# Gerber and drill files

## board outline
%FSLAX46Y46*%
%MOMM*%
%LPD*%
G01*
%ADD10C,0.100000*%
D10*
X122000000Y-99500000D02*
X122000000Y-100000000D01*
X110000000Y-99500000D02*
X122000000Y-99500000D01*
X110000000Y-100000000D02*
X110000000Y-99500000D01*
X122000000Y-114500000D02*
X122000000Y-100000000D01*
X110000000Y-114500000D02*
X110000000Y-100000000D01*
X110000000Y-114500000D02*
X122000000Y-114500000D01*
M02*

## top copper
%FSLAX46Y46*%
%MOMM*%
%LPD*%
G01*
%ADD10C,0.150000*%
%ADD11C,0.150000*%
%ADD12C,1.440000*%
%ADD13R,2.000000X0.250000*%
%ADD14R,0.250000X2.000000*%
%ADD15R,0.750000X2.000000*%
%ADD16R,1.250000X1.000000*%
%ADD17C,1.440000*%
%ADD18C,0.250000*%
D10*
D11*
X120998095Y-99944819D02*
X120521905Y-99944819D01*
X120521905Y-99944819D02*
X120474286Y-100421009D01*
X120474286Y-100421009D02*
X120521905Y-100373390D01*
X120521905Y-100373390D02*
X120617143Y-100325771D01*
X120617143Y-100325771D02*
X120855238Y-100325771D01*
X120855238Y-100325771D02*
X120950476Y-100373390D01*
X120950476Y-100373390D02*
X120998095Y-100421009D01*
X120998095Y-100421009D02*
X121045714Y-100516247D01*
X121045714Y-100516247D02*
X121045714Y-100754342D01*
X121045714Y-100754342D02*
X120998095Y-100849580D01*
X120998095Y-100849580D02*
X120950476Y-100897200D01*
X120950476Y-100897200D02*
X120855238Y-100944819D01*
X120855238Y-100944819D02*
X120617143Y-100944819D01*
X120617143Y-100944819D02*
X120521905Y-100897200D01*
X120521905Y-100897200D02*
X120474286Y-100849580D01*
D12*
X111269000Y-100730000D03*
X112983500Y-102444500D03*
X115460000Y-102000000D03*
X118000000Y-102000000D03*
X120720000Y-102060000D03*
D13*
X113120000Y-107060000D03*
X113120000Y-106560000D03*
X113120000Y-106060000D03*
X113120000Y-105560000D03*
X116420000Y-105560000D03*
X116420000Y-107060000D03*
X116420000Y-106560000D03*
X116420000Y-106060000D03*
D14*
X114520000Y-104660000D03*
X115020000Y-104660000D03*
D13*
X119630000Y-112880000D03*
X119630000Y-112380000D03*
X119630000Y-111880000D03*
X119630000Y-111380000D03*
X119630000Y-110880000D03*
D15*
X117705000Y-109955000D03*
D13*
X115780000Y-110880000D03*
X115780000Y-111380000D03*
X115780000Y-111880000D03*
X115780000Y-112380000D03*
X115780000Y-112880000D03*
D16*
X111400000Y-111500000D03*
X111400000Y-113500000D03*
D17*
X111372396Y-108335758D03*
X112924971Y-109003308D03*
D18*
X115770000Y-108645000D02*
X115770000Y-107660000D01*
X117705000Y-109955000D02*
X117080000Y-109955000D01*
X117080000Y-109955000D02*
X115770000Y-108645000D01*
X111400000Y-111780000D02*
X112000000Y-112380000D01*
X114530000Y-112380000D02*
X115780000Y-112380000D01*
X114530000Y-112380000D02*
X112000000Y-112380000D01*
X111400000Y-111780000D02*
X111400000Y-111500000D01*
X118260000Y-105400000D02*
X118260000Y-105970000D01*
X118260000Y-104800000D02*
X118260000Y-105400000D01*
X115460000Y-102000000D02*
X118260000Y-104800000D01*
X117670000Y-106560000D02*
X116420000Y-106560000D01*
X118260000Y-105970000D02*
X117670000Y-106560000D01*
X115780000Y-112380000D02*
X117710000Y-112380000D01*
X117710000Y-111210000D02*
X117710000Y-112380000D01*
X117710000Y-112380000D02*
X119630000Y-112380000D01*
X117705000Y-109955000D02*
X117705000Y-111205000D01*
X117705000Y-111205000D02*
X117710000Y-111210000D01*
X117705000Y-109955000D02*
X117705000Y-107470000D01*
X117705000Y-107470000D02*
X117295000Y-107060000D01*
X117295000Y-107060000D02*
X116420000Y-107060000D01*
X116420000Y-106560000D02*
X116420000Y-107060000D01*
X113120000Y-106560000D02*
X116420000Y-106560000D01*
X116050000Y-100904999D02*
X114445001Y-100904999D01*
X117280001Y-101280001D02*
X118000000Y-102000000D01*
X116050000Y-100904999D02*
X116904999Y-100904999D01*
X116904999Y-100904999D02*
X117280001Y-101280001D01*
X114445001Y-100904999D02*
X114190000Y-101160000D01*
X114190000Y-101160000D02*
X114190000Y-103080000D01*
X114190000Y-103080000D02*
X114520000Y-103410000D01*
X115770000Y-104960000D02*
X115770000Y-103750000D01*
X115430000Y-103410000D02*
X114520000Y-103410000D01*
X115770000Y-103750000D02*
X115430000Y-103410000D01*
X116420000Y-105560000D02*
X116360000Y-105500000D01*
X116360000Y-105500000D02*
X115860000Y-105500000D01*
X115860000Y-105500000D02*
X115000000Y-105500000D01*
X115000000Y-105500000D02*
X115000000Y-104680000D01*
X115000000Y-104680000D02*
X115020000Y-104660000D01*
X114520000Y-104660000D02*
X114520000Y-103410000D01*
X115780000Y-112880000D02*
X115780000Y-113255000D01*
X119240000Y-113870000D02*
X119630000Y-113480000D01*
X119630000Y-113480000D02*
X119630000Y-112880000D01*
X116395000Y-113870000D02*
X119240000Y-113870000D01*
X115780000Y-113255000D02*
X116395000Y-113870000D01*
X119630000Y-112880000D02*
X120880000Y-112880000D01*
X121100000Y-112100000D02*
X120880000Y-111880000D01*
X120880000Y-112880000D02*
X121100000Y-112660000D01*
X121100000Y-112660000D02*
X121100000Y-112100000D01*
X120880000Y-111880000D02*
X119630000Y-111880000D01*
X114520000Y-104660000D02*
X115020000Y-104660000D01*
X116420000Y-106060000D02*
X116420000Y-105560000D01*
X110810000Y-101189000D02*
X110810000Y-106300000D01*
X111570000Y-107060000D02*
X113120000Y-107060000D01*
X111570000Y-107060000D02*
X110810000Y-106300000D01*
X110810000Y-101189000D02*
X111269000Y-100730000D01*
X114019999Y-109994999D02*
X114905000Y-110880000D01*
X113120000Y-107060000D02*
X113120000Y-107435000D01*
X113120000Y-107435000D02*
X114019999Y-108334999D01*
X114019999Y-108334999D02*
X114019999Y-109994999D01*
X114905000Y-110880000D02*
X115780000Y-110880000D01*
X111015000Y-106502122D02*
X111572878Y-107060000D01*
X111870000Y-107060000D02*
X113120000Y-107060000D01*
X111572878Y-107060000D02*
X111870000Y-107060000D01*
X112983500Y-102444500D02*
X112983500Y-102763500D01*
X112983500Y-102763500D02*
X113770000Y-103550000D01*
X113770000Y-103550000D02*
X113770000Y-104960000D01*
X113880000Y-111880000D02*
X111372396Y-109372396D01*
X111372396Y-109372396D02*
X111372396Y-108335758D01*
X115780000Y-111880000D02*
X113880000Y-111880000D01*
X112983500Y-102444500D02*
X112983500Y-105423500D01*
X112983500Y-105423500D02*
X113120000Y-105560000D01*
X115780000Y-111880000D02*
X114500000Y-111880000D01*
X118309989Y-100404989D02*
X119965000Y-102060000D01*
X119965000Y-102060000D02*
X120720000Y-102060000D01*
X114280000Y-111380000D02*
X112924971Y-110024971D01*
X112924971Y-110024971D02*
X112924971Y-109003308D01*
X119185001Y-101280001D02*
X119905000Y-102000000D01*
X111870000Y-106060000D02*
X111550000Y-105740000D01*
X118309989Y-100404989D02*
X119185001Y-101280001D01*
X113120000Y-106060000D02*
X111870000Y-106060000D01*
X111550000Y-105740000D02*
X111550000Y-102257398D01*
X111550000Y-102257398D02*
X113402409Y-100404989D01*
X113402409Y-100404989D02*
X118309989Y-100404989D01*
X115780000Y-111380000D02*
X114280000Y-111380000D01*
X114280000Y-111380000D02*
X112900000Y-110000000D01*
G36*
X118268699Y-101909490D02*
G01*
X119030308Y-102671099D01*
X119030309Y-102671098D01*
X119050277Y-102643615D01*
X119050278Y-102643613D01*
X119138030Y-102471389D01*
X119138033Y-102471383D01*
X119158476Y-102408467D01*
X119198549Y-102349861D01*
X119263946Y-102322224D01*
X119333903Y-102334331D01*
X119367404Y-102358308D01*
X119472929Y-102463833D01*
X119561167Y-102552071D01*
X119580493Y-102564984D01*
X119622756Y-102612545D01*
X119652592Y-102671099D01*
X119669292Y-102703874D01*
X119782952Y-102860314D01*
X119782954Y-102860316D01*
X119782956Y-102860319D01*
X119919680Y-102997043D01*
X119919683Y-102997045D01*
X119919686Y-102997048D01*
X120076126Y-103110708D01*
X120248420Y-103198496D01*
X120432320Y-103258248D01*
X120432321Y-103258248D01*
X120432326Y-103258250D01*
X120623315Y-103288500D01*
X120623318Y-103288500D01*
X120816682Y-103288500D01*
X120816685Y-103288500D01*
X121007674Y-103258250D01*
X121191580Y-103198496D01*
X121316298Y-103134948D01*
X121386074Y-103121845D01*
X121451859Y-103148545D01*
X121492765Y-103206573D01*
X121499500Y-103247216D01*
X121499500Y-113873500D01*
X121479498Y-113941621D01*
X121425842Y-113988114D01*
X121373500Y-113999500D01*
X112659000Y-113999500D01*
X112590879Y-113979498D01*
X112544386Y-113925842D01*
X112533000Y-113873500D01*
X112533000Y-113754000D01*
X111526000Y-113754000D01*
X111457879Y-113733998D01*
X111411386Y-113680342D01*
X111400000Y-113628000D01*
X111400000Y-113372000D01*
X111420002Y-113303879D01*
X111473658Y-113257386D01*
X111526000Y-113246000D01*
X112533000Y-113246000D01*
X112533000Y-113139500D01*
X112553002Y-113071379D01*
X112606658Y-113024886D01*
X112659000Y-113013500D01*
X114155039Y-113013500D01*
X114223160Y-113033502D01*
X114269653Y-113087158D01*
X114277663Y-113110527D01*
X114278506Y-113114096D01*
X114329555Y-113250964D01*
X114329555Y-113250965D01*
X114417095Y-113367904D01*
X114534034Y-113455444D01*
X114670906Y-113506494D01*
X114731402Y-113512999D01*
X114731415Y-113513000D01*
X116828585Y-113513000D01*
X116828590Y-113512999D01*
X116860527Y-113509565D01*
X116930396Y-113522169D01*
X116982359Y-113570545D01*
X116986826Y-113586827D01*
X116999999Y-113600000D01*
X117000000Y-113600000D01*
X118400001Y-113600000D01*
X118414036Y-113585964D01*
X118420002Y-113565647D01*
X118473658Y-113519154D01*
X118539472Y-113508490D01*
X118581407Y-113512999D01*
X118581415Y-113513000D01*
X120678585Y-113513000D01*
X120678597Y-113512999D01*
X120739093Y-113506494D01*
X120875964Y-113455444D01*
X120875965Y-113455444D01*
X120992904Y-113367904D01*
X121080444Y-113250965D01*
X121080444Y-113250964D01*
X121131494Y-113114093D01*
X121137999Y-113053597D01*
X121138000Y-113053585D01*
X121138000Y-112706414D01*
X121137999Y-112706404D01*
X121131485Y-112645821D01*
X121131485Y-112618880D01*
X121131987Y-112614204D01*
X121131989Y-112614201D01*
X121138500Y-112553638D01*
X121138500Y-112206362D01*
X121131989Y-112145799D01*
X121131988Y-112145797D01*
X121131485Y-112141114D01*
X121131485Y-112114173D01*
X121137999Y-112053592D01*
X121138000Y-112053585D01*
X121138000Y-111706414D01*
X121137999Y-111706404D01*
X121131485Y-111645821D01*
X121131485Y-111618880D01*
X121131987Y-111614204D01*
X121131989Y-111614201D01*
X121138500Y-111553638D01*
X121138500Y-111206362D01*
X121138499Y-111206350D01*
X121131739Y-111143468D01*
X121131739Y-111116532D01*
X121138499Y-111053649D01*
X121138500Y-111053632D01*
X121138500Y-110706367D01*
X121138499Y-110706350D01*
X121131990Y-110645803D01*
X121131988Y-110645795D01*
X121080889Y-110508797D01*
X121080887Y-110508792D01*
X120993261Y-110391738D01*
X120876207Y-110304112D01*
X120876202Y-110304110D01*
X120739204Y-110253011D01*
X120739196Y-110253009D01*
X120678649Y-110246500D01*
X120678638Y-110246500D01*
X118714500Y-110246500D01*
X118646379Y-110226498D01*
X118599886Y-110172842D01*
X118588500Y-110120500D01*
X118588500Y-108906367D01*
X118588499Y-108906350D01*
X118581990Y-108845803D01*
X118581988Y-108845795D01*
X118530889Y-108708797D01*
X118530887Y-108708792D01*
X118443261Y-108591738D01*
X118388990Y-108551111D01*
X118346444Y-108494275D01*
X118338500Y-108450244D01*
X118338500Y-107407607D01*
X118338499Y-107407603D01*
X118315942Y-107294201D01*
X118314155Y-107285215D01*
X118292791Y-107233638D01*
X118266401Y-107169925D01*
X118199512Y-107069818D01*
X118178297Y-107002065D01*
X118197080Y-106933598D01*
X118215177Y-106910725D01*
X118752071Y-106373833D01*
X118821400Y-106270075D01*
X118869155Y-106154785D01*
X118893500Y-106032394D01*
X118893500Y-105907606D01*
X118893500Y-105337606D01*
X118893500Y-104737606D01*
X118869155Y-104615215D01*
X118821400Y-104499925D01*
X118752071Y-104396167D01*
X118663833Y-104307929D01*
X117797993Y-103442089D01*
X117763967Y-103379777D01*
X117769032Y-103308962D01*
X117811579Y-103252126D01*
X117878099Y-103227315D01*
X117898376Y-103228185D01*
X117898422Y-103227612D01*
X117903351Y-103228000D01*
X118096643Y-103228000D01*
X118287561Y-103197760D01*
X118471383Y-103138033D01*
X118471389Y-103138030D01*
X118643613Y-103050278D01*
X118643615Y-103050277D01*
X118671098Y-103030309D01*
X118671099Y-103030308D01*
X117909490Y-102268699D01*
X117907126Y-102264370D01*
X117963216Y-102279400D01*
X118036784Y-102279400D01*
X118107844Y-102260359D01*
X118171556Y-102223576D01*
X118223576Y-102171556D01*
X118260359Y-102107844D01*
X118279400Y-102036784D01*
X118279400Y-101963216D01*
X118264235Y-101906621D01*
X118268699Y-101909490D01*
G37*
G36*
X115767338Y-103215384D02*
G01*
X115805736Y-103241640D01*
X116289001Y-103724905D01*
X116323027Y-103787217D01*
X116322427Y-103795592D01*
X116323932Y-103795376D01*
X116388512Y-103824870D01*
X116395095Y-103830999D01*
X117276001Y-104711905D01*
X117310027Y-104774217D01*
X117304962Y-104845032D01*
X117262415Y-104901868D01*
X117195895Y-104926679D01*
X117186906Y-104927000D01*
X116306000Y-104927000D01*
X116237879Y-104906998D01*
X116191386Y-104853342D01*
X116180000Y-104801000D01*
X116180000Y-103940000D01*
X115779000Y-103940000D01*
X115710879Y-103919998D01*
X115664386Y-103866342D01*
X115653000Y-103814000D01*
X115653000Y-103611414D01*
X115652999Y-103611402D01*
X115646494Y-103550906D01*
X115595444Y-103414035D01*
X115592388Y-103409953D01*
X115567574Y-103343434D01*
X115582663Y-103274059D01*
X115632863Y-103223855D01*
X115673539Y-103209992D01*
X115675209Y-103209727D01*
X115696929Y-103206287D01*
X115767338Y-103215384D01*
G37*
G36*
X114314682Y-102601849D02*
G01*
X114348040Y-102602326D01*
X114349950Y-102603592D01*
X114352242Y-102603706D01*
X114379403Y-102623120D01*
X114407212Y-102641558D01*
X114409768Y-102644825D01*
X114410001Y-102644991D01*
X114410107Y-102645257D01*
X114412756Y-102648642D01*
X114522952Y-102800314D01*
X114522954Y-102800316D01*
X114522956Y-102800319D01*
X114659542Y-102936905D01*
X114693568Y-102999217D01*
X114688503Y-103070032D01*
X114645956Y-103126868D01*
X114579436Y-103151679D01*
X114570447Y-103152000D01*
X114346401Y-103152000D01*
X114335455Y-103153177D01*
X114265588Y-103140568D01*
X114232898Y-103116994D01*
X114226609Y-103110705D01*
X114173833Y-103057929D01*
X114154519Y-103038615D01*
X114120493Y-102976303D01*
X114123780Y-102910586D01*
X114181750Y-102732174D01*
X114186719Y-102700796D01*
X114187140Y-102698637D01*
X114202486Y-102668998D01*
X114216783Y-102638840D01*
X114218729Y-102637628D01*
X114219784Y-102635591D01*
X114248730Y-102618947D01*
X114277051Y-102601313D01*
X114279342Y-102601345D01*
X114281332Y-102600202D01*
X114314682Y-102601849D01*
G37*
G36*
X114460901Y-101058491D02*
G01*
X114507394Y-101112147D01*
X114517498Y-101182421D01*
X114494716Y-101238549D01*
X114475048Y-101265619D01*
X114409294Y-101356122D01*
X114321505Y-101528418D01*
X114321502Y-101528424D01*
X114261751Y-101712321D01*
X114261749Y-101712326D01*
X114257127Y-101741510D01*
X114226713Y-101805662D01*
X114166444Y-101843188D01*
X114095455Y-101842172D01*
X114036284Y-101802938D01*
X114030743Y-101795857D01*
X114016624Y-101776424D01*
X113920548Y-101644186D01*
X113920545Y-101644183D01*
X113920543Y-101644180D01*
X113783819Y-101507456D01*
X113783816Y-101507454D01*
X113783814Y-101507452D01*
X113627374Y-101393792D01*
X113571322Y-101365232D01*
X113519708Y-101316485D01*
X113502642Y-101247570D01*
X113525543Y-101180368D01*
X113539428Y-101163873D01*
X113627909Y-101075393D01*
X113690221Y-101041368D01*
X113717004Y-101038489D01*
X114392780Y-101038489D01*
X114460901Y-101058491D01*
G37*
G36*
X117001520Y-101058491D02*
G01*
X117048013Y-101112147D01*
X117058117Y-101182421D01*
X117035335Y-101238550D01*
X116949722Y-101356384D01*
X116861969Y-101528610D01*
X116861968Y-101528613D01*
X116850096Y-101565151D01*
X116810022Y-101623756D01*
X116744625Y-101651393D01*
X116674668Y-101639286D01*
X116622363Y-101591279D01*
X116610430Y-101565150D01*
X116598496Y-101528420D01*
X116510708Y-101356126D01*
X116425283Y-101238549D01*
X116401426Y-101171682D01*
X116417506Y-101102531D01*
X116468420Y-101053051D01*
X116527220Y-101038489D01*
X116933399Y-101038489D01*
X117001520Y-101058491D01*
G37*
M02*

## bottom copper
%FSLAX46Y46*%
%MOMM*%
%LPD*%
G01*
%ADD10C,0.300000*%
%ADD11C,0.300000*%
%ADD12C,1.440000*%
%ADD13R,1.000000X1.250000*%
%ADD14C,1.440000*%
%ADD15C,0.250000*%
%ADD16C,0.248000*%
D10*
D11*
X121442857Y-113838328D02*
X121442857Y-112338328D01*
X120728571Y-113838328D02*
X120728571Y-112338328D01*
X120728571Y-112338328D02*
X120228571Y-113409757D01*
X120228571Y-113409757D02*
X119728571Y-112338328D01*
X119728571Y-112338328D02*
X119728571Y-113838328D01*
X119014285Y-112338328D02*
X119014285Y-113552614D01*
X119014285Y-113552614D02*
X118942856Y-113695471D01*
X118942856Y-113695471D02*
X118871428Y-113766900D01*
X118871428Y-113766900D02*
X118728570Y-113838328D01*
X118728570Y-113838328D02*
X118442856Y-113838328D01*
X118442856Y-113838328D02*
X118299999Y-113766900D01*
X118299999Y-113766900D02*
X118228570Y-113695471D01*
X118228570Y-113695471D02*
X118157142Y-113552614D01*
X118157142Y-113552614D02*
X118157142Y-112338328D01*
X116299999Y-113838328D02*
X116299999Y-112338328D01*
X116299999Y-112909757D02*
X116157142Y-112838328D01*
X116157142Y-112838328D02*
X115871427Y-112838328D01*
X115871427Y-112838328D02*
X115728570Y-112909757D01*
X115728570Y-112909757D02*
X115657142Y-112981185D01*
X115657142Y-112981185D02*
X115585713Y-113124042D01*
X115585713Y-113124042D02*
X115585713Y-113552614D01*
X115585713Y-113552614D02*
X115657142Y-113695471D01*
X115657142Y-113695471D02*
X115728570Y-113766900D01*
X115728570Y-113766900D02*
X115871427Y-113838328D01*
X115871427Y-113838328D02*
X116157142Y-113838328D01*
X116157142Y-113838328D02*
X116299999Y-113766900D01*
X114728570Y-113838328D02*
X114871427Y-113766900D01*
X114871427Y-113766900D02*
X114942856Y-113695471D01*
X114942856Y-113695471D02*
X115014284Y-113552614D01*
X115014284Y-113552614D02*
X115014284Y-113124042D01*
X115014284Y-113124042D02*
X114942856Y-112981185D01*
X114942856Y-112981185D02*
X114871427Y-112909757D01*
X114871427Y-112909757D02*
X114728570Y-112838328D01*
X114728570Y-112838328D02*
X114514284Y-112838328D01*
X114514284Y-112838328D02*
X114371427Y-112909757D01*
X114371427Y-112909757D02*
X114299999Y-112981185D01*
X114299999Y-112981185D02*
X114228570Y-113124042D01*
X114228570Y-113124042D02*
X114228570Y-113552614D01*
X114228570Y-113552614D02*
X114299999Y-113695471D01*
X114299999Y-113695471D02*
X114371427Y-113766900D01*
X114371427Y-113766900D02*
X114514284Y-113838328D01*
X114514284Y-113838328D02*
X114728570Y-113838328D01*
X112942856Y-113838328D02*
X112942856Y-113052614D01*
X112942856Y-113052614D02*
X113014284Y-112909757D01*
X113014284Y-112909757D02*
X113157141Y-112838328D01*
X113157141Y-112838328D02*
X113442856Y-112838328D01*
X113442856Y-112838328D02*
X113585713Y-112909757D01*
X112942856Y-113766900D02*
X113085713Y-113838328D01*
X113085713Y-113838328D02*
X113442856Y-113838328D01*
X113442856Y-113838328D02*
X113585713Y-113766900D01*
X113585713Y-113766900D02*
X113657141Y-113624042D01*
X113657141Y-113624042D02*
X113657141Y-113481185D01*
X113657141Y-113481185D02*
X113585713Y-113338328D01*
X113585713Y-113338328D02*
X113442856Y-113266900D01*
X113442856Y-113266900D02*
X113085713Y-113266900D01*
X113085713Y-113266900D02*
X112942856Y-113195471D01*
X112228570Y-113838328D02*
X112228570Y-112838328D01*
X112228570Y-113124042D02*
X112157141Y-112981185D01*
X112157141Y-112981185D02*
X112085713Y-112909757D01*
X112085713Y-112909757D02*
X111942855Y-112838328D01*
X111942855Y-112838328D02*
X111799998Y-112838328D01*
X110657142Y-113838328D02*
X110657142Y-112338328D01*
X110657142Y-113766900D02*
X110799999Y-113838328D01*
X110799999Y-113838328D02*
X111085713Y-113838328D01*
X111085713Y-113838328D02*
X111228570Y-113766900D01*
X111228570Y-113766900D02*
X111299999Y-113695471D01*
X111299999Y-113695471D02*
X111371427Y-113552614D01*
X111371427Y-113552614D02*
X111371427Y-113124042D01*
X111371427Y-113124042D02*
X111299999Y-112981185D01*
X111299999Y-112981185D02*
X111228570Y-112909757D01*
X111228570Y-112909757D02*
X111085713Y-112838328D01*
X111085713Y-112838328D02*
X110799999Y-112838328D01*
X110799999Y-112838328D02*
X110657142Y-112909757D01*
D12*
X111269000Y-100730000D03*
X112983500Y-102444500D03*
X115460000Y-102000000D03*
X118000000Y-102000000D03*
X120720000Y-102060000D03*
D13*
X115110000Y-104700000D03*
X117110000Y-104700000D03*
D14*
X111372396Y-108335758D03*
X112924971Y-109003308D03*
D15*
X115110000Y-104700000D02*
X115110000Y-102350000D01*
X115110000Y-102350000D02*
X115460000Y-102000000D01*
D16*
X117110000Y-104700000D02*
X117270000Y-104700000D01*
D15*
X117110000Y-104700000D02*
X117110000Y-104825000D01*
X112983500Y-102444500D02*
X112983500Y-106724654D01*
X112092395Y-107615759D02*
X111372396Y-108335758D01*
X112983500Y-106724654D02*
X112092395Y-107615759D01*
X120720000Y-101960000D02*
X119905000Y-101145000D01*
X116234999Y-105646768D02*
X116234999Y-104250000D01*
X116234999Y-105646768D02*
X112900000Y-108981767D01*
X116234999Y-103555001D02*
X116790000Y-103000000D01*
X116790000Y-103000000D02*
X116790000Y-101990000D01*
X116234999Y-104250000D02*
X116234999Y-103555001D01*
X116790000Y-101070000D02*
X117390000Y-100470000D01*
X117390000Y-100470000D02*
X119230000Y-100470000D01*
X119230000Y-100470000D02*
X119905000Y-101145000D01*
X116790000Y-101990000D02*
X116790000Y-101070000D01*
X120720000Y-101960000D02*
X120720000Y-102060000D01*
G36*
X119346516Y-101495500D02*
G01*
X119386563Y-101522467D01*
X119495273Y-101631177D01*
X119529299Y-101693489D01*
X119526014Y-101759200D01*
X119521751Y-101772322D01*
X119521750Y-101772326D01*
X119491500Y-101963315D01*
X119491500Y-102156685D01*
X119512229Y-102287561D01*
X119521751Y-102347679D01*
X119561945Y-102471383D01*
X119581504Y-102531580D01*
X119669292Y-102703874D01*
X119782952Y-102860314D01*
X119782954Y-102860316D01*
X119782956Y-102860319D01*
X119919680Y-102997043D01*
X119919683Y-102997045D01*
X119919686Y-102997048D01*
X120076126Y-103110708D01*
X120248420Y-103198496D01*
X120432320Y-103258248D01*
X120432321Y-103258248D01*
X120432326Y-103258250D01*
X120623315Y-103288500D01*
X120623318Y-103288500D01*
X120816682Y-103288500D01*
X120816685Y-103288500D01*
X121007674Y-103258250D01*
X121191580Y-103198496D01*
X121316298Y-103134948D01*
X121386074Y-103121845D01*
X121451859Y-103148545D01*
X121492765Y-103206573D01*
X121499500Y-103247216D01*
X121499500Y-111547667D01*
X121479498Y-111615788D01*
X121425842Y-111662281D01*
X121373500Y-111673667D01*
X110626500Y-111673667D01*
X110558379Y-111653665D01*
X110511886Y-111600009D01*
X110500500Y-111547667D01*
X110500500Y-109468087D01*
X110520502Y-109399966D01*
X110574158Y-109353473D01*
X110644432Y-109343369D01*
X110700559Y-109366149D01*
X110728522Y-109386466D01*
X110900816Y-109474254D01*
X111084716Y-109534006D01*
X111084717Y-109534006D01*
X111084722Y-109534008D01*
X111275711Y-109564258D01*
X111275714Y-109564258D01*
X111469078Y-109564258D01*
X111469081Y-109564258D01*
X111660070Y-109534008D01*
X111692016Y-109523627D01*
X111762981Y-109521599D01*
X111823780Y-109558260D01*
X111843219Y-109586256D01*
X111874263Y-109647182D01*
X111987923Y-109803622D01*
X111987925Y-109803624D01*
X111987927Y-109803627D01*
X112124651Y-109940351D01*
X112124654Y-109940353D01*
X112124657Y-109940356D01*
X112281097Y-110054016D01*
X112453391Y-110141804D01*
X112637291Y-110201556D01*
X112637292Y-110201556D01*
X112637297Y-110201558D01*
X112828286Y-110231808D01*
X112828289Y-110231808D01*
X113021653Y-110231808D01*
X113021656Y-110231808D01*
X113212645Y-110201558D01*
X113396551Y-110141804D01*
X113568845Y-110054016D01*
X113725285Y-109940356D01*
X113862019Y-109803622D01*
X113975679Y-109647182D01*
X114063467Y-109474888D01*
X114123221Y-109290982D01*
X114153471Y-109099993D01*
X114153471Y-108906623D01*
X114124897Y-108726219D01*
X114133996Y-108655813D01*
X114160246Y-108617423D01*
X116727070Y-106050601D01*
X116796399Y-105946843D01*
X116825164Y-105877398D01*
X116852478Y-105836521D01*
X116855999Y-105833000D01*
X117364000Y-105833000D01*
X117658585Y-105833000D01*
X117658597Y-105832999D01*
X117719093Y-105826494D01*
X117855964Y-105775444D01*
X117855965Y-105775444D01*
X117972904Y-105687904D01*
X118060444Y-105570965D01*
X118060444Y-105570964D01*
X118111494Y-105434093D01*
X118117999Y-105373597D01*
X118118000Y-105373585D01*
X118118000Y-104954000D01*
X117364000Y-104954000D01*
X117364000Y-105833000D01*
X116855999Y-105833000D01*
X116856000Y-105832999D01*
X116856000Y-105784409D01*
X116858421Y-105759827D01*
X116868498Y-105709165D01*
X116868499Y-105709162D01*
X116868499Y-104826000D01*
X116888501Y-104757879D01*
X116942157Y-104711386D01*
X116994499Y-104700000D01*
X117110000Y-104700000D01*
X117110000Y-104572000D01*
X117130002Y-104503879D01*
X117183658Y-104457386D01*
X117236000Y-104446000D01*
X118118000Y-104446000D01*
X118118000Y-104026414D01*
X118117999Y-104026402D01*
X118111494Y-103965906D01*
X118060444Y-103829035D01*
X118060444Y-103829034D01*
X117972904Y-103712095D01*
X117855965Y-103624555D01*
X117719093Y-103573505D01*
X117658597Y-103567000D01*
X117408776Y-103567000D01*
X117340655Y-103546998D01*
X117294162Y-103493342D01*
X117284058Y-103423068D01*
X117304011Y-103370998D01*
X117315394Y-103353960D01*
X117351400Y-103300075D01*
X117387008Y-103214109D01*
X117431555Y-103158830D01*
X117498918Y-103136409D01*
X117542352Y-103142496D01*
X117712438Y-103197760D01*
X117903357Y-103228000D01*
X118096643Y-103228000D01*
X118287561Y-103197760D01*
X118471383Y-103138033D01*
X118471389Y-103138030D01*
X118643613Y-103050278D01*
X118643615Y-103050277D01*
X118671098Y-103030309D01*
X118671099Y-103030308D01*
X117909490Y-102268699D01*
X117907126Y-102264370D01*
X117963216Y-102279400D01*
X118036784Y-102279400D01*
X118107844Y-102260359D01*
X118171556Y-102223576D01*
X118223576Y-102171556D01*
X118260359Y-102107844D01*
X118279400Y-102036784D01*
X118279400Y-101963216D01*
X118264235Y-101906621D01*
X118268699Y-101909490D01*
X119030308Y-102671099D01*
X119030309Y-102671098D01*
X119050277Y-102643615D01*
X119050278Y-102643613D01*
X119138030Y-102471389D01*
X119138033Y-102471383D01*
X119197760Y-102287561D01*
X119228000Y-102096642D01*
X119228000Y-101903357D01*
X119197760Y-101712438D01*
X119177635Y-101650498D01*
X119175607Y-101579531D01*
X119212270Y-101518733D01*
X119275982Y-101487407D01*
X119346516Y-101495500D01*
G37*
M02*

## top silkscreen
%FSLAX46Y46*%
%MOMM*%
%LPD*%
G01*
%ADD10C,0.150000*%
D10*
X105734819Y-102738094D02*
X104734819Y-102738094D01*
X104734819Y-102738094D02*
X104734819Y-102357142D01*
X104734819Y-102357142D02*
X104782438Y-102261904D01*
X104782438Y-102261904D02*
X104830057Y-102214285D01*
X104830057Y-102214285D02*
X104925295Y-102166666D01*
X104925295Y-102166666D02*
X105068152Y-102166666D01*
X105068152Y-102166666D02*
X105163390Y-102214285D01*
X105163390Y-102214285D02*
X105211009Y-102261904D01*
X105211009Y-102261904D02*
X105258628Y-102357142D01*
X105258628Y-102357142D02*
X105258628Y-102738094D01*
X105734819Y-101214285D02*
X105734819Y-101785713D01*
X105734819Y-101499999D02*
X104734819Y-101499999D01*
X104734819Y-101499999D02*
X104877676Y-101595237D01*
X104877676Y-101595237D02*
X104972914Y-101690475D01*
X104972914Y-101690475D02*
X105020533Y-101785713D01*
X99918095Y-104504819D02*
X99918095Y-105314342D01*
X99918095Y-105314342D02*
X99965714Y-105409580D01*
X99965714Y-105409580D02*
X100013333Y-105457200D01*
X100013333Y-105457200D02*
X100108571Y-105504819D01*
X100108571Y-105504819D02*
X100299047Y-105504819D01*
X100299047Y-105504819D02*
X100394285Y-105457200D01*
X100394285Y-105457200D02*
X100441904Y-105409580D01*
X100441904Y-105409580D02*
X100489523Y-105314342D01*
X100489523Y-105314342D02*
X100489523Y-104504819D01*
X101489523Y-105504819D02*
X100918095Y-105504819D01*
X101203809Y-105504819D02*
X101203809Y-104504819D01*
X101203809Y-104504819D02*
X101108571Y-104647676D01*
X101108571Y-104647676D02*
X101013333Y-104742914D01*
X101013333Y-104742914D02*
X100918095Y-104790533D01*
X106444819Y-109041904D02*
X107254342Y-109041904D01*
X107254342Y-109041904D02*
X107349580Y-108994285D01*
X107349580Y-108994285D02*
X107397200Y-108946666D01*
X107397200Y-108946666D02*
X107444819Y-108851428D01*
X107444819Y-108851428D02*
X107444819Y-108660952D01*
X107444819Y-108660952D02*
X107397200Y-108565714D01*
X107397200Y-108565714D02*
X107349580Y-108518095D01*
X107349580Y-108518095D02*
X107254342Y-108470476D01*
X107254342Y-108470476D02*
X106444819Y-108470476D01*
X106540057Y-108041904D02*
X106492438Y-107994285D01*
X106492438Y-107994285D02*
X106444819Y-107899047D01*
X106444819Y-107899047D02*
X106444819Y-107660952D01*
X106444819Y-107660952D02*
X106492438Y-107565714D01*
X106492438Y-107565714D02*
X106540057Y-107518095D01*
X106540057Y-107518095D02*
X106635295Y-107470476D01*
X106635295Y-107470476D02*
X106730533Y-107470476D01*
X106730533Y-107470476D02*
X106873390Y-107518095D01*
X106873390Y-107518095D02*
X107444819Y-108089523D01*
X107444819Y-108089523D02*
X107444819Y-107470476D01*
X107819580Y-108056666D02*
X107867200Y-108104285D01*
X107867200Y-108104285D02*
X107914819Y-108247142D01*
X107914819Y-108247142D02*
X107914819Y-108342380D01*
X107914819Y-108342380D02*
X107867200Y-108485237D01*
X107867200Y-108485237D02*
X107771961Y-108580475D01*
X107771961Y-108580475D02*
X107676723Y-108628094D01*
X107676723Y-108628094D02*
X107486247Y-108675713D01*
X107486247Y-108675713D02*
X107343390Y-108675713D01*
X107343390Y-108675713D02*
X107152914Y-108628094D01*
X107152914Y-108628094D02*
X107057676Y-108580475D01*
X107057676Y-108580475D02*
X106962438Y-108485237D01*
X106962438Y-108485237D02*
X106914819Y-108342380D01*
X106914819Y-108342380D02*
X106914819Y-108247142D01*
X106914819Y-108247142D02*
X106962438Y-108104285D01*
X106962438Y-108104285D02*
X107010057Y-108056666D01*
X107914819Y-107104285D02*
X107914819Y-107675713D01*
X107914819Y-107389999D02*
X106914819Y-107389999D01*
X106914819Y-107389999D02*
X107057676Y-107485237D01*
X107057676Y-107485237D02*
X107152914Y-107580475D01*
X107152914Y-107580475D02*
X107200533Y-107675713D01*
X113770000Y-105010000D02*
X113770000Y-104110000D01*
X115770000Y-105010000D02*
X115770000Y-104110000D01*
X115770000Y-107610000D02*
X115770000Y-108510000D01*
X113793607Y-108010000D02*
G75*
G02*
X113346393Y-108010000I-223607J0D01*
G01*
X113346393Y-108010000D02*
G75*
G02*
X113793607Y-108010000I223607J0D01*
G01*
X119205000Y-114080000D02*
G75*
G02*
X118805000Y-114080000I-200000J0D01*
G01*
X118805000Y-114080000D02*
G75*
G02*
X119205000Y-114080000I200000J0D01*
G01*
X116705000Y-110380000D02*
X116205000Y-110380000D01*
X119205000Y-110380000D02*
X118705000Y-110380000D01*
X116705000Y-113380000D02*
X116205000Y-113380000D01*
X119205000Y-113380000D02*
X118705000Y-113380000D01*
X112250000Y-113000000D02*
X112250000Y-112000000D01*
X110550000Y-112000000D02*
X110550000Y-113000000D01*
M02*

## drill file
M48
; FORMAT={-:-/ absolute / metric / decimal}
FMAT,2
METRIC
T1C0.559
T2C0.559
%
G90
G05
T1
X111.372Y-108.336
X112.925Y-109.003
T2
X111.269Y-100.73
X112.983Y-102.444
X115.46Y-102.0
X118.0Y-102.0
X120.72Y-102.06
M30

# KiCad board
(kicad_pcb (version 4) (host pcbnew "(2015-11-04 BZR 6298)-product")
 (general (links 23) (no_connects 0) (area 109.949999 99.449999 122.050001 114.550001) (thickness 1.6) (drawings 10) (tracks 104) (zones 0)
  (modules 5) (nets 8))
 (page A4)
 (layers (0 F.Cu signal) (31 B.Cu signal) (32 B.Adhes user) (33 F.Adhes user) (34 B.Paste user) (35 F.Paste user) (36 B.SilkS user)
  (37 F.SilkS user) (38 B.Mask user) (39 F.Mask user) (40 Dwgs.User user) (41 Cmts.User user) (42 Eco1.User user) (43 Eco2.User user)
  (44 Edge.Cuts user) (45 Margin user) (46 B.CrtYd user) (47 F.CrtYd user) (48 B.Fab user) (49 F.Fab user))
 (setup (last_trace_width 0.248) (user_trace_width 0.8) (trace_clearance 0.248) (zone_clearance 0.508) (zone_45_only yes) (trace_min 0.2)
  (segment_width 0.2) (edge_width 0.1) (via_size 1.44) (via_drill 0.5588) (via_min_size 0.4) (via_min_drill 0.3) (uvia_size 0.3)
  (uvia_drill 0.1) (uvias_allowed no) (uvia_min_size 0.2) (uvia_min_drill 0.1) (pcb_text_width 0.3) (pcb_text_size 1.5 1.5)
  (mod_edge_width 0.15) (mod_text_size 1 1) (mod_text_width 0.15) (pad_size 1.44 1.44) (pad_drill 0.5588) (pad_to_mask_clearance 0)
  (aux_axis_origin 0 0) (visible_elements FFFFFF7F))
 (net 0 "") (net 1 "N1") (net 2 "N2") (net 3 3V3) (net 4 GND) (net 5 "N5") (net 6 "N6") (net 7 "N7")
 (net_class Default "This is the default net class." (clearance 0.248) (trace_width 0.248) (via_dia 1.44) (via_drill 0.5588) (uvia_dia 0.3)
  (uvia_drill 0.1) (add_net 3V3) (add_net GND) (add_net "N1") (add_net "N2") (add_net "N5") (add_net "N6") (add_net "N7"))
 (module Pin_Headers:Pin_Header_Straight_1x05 (layer F.Cu) (at 110.38 102 90)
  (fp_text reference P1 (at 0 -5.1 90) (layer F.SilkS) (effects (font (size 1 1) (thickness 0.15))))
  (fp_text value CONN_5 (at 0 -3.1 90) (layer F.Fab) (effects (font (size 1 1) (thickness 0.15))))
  (pad 1 thru_hole circle (at 1.27 0.889 90) (size 1.44 1.44) (drill 0.5588) (layers *.Cu *.Mask) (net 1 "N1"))
  (pad 2 thru_hole circle (at -0.4445 2.6035 90) (size 1.44 1.44) (drill 0.5588) (layers *.Cu *.Mask) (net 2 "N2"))
  (pad 3 thru_hole circle (at 0 5.08 90) (size 1.44 1.44) (drill 0.5588) (layers *.Cu *.Mask) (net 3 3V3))
  (pad 4 thru_hole circle (at 0 7.62 90) (size 1.44 1.44) (drill 0.5588) (layers *.Cu *.Mask) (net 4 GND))
  (pad 5 thru_hole circle (at -0.06 10.34 90) (size 1.44 1.44) (drill 0.5588) (layers *.Cu *.Mask) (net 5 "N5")))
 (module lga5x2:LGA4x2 (layer F.Cu) (at 114.77 106.31 180)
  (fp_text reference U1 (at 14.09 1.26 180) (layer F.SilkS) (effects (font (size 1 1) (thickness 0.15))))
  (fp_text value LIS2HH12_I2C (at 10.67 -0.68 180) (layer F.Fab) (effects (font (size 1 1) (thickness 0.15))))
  (fp_line (start 1 1.3) (end 1 2.2) (layer F.SilkS) (width 0.15))
  (fp_line (start -1 1.3) (end -1 2.2) (layer F.SilkS) (width 0.15))
  (fp_line (start -1 -1.3) (end -1 -2.2) (layer F.SilkS) (width 0.15))
  (fp_circle (center 1.2 -1.7) (end 1.1 -1.9) (layer F.SilkS) (width 0.15))
  (pad 1 smd rect (at 1.65 -0.75 180) (size 2 0.25) (layers F.Cu F.Paste F.Mask) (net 1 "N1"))
  (pad 2 smd rect (at 1.65 -0.25 180) (size 2 0.25) (layers F.Cu F.Paste F.Mask) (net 3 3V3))
  (pad 3 smd rect (at 1.65 0.25 180) (size 2 0.25) (layers F.Cu F.Paste F.Mask) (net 5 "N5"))
  (pad 4 smd rect (at 1.65 0.75 180) (size 2 0.25) (layers F.Cu F.Paste F.Mask) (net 2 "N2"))
  (pad 7 smd rect (at -1.65 0.75 180) (size 2 0.25) (layers F.Cu F.Paste F.Mask) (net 4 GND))
  (pad 10 smd rect (at -1.65 -0.75 180) (size 2 0.25) (layers F.Cu F.Paste F.Mask) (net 3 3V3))
  (pad 9 smd rect (at -1.65 -0.25 180) (size 2 0.25) (layers F.Cu F.Paste F.Mask) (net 3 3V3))
  (pad 8 smd rect (at -1.65 0.25 180) (size 2 0.25) (layers F.Cu F.Paste F.Mask) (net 4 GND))
  (pad 5 smd rect (at 0.25 1.65 180) (size 0.25 2) (layers F.Cu F.Paste F.Mask) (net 4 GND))
  (pad 6 smd rect (at -0.25 1.65 180) (size 0.25 2) (layers F.Cu F.Paste F.Mask) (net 4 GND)))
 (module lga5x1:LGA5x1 (layer F.Cu) (at 117.705 111.88 270)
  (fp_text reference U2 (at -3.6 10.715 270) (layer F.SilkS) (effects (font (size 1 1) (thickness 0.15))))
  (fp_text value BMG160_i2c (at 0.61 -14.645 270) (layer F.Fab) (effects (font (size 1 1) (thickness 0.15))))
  (fp_circle (center 2.2 -1.3) (end 2.2 -1.5) (layer F.SilkS) (width 0.15))
  (fp_line (start -1.5 1) (end -1.5 1.5) (layer F.SilkS) (width 0.15))
  (fp_line (start -1.5 -1.5) (end -1.5 -1) (layer F.SilkS) (width 0.15))
  (fp_line (start 1.5 1) (end 1.5 1.5) (layer F.SilkS) (width 0.15))
  (fp_line (start 1.5 -1.5) (end 1.5 -1) (layer F.SilkS) (width 0.15))
  (pad 1 smd rect (at 1 -1.925 270) (size 0.25 2) (layers F.Cu F.Paste F.Mask) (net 4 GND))
  (pad 2 smd rect (at 0.5 -1.925 270) (size 0.25 2) (layers F.Cu F.Paste F.Mask) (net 3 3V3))
  (pad 3 smd rect (at 0 -1.925 270) (size 0.25 2) (layers F.Cu F.Paste F.Mask) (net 4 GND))
  (pad 4 smd rect (at -0.5 -1.925 270) (size 0.25 2) (layers F.Cu F.Paste F.Mask) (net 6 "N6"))
  (pad 5 smd rect (at -1 -1.925 270) (size 0.25 2) (layers F.Cu F.Paste F.Mask) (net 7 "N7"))
  (pad 6 smd rect (at -1.925 0 270) (size 2 0.75) (layers F.Cu F.Paste F.Mask) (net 3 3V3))
  (pad 7 smd rect (at -1 1.925 270) (size 0.25 2) (layers F.Cu F.Paste F.Mask) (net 1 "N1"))
  (pad 8 smd rect (at -0.5 1.925 270) (size 0.25 2) (layers F.Cu F.Paste F.Mask) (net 5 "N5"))
  (pad 9 smd rect (at 0 1.925 270) (size 0.25 2) (layers F.Cu F.Paste F.Mask) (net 2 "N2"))
  (pad 10 smd rect (at 0.5 1.925 270) (size 0.25 2) (layers F.Cu F.Paste F.Mask) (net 3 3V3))
  (pad 11 smd rect (at 1 1.925 270) (size 0.25 2) (layers F.Cu F.Paste F.Mask) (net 4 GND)))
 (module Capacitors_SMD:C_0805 (layer F.Cu) (at 111.4 112.5 270)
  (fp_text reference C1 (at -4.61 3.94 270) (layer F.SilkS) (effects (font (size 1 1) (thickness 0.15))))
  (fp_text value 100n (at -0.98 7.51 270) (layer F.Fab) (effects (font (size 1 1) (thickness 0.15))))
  (fp_line (start 0.5 -0.85) (end -0.5 -0.85) (layer F.SilkS) (width 0.15))
  (fp_line (start -0.5 0.85) (end 0.5 0.85) (layer F.SilkS) (width 0.15))
  (pad 1 smd rect (at -1 0 270) (size 1 1.25) (layers F.Cu F.Paste F.Mask) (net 3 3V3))
  (pad 2 smd rect (at 1 0 270) (size 1 1.25) (layers F.Cu F.Paste F.Mask) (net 4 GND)))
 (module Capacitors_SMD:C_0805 (layer B.Cu) (at 116.11 104.7)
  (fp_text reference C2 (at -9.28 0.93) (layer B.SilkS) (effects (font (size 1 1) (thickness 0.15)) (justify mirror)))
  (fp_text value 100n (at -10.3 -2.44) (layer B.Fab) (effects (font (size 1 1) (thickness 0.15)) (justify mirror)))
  (pad 1 smd rect (at -1 0) (size 1 1.25) (layers B.Cu B.Paste B.Mask) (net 3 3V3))
  (pad 2 smd rect (at 1 0) (size 1 1.25) (layers B.Cu B.Paste B.Mask) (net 4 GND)))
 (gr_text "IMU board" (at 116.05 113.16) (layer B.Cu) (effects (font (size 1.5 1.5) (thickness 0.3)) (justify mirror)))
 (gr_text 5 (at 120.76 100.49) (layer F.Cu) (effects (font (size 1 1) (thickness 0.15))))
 (gr_line (start 122 99.5) (end 122 100) (angle 90) (layer Edge.Cuts) (width 0.1))
 (gr_line (start 110 99.5) (end 122 99.5) (angle 90) (layer Edge.Cuts) (width 0.1))
 (gr_line (start 110 100) (end 110 99.5) (angle 90) (layer Edge.Cuts) (width 0.1))
 (gr_line (start 122 114.5) (end 122 100) (angle 90) (layer Edge.Cuts) (width 0.1))
 (gr_line (start 110 114.5) (end 110 100) (angle 90) (layer Edge.Cuts) (width 0.1))
 (gr_line (start 110 114.5) (end 122 114.5) (angle 90) (layer Edge.Cuts) (width 0.1))
 (segment (start 115.77 108.645) (end 115.77 107.66) (width 0.25) (layer F.Cu) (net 3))
 (segment (start 117.705 109.955) (end 117.08 109.955) (width 0.25) (layer F.Cu) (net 3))
 (segment (start 117.08 109.955) (end 115.77 108.645) (width 0.25) (layer F.Cu) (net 3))
 (segment (start 111.4 111.78) (end 112 112.38) (width 0.25) (layer F.Cu) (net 3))
 (segment (start 114.53 112.38) (end 115.78 112.38) (width 0.25) (layer F.Cu) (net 3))
 (segment (start 114.53 112.38) (end 112 112.38) (width 0.25) (layer F.Cu) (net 3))
 (segment (start 111.4 111.78) (end 111.4 111.5) (width 0.25) (layer F.Cu) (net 3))
 (segment (start 118.26 105.4) (end 118.26 105.97) (width 0.25) (layer F.Cu) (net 3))
 (segment (start 118.26 104.8) (end 118.26 105.4) (width 0.25) (layer F.Cu) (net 3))
 (segment (start 115.11 104.7) (end 115.11 102.35) (width 0.25) (layer B.Cu) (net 3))
 (segment (start 115.11 102.35) (end 115.46 102) (width 0.25) (layer B.Cu) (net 3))
 (segment (start 115.46 102) (end 118.26 104.8) (width 0.25) (layer F.Cu) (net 3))
 (segment (start 117.67 106.56) (end 116.42 106.56) (width 0.25) (layer F.Cu) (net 3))
 (segment (start 118.26 105.97) (end 117.67 106.56) (width 0.25) (layer F.Cu) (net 3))
 (segment (start 115.78 112.38) (end 117.71 112.38) (width 0.25) (layer F.Cu) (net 3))
 (segment (start 117.71 111.21) (end 117.71 112.38) (width 0.25) (layer F.Cu) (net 3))
 (segment (start 117.71 112.38) (end 119.63 112.38) (width 0.25) (layer F.Cu) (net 3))
 (segment (start 117.705 109.955) (end 117.705 111.205) (width 0.25) (layer F.Cu) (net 3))
 (segment (start 117.705 111.205) (end 117.71 111.21) (width 0.25) (layer F.Cu) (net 3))
 (segment (start 117.705 109.955) (end 117.705 107.47) (width 0.25) (layer F.Cu) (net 3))
 (segment (start 117.705 107.47) (end 117.295 107.06) (width 0.25) (layer F.Cu) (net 3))
 (segment (start 117.295 107.06) (end 116.42 107.06) (width 0.25) (layer F.Cu) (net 3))
 (segment (start 116.42 106.56) (end 116.42 107.06) (width 0.25) (layer F.Cu) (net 3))
 (segment (start 113.12 106.56) (end 116.42 106.56) (width 0.25) (layer F.Cu) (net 3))
 (segment (start 117.11 104.7) (end 117.27 104.7) (width 0.248) (layer B.Cu) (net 4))
 (segment (start 116.05 100.904999) (end 114.445001 100.904999) (width 0.25) (layer F.Cu) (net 4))
 (segment (start 117.280001 101.280001) (end 118 102) (width 0.25) (layer F.Cu) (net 4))
 (segment (start 116.05 100.904999) (end 116.904999 100.904999) (width 0.25) (layer F.Cu) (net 4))
 (segment (start 116.904999 100.904999) (end 117.280001 101.280001) (width 0.25) (layer F.Cu) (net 4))
 (segment (start 114.445001 100.904999) (end 114.19 101.16) (width 0.25) (layer F.Cu) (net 4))
 (segment (start 114.19 101.16) (end 114.19 103.08) (width 0.25) (layer F.Cu) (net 4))
 (segment (start 114.19 103.08) (end 114.52 103.41) (width 0.25) (layer F.Cu) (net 4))
 (segment (start 115.77 104.96) (end 115.77 103.75) (width 0.25) (layer F.Cu) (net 4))
 (segment (start 115.43 103.41) (end 114.52 103.41) (width 0.25) (layer F.Cu) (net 4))
 (segment (start 115.77 103.75) (end 115.43 103.41) (width 0.25) (layer F.Cu) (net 4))
 (segment (start 116.42 105.56) (end 116.36 105.5) (width 0.25) (layer F.Cu) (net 4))
 (segment (start 116.36 105.5) (end 115.86 105.5) (width 0.25) (layer F.Cu) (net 4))
 (segment (start 115.86 105.5) (end 115 105.5) (width 0.25) (layer F.Cu) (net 4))
 (segment (start 115 105.5) (end 115 104.68) (width 0.25) (layer F.Cu) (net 4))
 (segment (start 115 104.68) (end 115.02 104.66) (width 0.25) (layer F.Cu) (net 4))
 (segment (start 114.52 104.66) (end 114.52 103.41) (width 0.25) (layer F.Cu) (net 4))
 (segment (start 117.11 104.7) (end 117.11 104.825) (width 0.25) (layer B.Cu) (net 4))
 (segment (start 115.78 112.88) (end 115.78 113.255) (width 0.25) (layer F.Cu) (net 4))
 (segment (start 119.24 113.87) (end 119.63 113.48) (width 0.25) (layer F.Cu) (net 4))
 (segment (start 119.63 113.48) (end 119.63 112.88) (width 0.25) (layer F.Cu) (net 4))
 (segment (start 116.395 113.87) (end 119.24 113.87) (width 0.25) (layer F.Cu) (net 4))
 (segment (start 115.78 113.255) (end 116.395 113.87) (width 0.25) (layer F.Cu) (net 4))
 (segment (start 119.63 112.88) (end 120.88 112.88) (width 0.25) (layer F.Cu) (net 4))
 (segment (start 121.1 112.1) (end 120.88 111.88) (width 0.25) (layer F.Cu) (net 4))
 (segment (start 120.88 112.88) (end 121.1 112.66) (width 0.25) (layer F.Cu) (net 4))
 (segment (start 121.1 112.66) (end 121.1 112.1) (width 0.25) (layer F.Cu) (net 4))
 (segment (start 120.88 111.88) (end 119.63 111.88) (width 0.25) (layer F.Cu) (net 4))
 (segment (start 114.52 104.66) (end 115.02 104.66) (width 0.25) (layer F.Cu) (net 4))
 (segment (start 116.42 106.06) (end 116.42 105.56) (width 0.25) (layer F.Cu) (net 4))
 (segment (start 110.81 101.189) (end 110.81 106.3) (width 0.25) (layer F.Cu) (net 1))
 (segment (start 111.57 107.06) (end 113.12 107.06) (width 0.25) (layer F.Cu) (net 1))
 (segment (start 111.57 107.06) (end 110.81 106.3) (width 0.25) (layer F.Cu) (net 1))
 (segment (start 110.81 101.189) (end 111.269 100.73) (width 0.25) (layer F.Cu) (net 1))
 (segment (start 114.019999 109.994999) (end 114.905 110.88) (width 0.25) (layer F.Cu) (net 1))
 (segment (start 113.12 107.06) (end 113.12 107.435) (width 0.25) (layer F.Cu) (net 1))
 (segment (start 113.12 107.435) (end 114.019999 108.334999) (width 0.25) (layer F.Cu) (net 1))
 (segment (start 114.019999 108.334999) (end 114.019999 109.994999) (width 0.25) (layer F.Cu) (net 1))
 (segment (start 114.905 110.88) (end 115.78 110.88) (width 0.25) (layer F.Cu) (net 1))
 (segment (start 111.015 106.502122) (end 111.572878 107.06) (width 0.25) (layer F.Cu) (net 1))
 (segment (start 111.87 107.06) (end 113.12 107.06) (width 0.25) (layer F.Cu) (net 1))
 (segment (start 111.572878 107.06) (end 111.87 107.06) (width 0.25) (layer F.Cu) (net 1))
 (segment (start 112.9835 102.4445) (end 112.9835 102.7635) (width 0.25) (layer F.Cu) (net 2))
 (segment (start 112.9835 102.7635) (end 113.77 103.55) (width 0.25) (layer F.Cu) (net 2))
 (segment (start 113.77 103.55) (end 113.77 104.96) (width 0.25) (layer F.Cu) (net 2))
 (segment (start 113.88 111.88) (end 111.372396 109.372396) (width 0.25) (layer F.Cu) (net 2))
 (segment (start 111.372396 109.372396) (end 111.372396 108.335758) (width 0.25) (layer F.Cu) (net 2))
 (segment (start 115.78 111.88) (end 113.88 111.88) (width 0.25) (layer F.Cu) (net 2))
 (segment (start 112.9835 102.4445) (end 112.9835 106.724654) (width 0.25) (layer B.Cu) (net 2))
 (via (at 111.372396 108.335758) (size 1.44) (drill 0.5588) (layers F.Cu B.Cu) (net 2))
 (segment (start 112.092395 107.615759) (end 111.372396 108.335758) (width 0.25) (layer B.Cu) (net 2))
 (segment (start 112.9835 106.724654) (end 112.092395 107.615759) (width 0.25) (layer B.Cu) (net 2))
 (segment (start 112.9835 102.4445) (end 112.9835 105.4235) (width 0.25) (layer F.Cu) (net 2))
 (segment (start 112.9835 105.4235) (end 113.12 105.56) (width 0.25) (layer F.Cu) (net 2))
 (segment (start 115.78 111.88) (end 114.5 111.88) (width 0.25) (layer F.Cu) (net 2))
 (segment (start 120.72 101.96) (end 119.905 101.145) (width 0.25) (layer B.Cu) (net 5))
 (segment (start 116.234999 105.646768) (end 116.234999 104.25) (width 0.25) (layer B.Cu) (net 5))
 (segment (start 116.234999 105.646768) (end 112.9 108.981767) (width 0.25) (layer B.Cu) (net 5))
 (via (at 112.924971 109.003308) (size 1.44) (drill 0.5588) (layers F.Cu B.Cu) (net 5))
 (segment (start 116.234999 103.555001) (end 116.79 103) (width 0.25) (layer B.Cu) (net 5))
 (segment (start 116.79 103) (end 116.79 101.99) (width 0.25) (layer B.Cu) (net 5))
 (segment (start 116.234999 104.25) (end 116.234999 103.555001) (width 0.25) (layer B.Cu) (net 5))
 (segment (start 116.79 101.07) (end 117.39 100.47) (width 0.25) (layer B.Cu) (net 5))
 (segment (start 117.39 100.47) (end 119.23 100.47) (width 0.25) (layer B.Cu) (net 5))
 (segment (start 119.23 100.47) (end 119.905 101.145) (width 0.25) (layer B.Cu) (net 5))
 (segment (start 116.79 101.99) (end 116.79 101.07) (width 0.25) (layer B.Cu) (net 5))
 (segment (start 120.72 101.96) (end 120.72 102.06) (width 0.25) (layer B.Cu) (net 5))
 (segment (start 118.309989 100.404989) (end 119.965 102.06) (width 0.25) (layer F.Cu) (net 5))
 (segment (start 119.965 102.06) (end 120.72 102.06) (width 0.25) (layer F.Cu) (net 5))
 (segment (start 114.28 111.38) (end 112.924971 110.024971) (width 0.25) (layer F.Cu) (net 5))
 (segment (start 112.924971 110.024971) (end 112.924971 109.003308) (width 0.25) (layer F.Cu) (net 5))
 (segment (start 119.185001 101.280001) (end 119.905 102) (width 0.25) (layer F.Cu) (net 5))
 (segment (start 111.87 106.06) (end 111.55 105.74) (width 0.25) (layer F.Cu) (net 5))
 (segment (start 118.309989 100.404989) (end 119.185001 101.280001) (width 0.25) (layer F.Cu) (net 5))
 (segment (start 113.12 106.06) (end 111.87 106.06) (width 0.25) (layer F.Cu) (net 5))
 (segment (start 111.55 105.74) (end 111.55 102.257398) (width 0.25) (layer F.Cu) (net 5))
 (segment (start 111.55 102.257398) (end 113.402409 100.404989) (width 0.25) (layer F.Cu) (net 5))
 (segment (start 113.402409 100.404989) (end 118.309989 100.404989) (width 0.25) (layer F.Cu) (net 5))
 (segment (start 115.78 111.38) (end 114.28 111.38) (width 0.25) (layer F.Cu) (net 5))
 (segment (start 114.28 111.38) (end 112.9 110) (width 0.25) (layer F.Cu) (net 5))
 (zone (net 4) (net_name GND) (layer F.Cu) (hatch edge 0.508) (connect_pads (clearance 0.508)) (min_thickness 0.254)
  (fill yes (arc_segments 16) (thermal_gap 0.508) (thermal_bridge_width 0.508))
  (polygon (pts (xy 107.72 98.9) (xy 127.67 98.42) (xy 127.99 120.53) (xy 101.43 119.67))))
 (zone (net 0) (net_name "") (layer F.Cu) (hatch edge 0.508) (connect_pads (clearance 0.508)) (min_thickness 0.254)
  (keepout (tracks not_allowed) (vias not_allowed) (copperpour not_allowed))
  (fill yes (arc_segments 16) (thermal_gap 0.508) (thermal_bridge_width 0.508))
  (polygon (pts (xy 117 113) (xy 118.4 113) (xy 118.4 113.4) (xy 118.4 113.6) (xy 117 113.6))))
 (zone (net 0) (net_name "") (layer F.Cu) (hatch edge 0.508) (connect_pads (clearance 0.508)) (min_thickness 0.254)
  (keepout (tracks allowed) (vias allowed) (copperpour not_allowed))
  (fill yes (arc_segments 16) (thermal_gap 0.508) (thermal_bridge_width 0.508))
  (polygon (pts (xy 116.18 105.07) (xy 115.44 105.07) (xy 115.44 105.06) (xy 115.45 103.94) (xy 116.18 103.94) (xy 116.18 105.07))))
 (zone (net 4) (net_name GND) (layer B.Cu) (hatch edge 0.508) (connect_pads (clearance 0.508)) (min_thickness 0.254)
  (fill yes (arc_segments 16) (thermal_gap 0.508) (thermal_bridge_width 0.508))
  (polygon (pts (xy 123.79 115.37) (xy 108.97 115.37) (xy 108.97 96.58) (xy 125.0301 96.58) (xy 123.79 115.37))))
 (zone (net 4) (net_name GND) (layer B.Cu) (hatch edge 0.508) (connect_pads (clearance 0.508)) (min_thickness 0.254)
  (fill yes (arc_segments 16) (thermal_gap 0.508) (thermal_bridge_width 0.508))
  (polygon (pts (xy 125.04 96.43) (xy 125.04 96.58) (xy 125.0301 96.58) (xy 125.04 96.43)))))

